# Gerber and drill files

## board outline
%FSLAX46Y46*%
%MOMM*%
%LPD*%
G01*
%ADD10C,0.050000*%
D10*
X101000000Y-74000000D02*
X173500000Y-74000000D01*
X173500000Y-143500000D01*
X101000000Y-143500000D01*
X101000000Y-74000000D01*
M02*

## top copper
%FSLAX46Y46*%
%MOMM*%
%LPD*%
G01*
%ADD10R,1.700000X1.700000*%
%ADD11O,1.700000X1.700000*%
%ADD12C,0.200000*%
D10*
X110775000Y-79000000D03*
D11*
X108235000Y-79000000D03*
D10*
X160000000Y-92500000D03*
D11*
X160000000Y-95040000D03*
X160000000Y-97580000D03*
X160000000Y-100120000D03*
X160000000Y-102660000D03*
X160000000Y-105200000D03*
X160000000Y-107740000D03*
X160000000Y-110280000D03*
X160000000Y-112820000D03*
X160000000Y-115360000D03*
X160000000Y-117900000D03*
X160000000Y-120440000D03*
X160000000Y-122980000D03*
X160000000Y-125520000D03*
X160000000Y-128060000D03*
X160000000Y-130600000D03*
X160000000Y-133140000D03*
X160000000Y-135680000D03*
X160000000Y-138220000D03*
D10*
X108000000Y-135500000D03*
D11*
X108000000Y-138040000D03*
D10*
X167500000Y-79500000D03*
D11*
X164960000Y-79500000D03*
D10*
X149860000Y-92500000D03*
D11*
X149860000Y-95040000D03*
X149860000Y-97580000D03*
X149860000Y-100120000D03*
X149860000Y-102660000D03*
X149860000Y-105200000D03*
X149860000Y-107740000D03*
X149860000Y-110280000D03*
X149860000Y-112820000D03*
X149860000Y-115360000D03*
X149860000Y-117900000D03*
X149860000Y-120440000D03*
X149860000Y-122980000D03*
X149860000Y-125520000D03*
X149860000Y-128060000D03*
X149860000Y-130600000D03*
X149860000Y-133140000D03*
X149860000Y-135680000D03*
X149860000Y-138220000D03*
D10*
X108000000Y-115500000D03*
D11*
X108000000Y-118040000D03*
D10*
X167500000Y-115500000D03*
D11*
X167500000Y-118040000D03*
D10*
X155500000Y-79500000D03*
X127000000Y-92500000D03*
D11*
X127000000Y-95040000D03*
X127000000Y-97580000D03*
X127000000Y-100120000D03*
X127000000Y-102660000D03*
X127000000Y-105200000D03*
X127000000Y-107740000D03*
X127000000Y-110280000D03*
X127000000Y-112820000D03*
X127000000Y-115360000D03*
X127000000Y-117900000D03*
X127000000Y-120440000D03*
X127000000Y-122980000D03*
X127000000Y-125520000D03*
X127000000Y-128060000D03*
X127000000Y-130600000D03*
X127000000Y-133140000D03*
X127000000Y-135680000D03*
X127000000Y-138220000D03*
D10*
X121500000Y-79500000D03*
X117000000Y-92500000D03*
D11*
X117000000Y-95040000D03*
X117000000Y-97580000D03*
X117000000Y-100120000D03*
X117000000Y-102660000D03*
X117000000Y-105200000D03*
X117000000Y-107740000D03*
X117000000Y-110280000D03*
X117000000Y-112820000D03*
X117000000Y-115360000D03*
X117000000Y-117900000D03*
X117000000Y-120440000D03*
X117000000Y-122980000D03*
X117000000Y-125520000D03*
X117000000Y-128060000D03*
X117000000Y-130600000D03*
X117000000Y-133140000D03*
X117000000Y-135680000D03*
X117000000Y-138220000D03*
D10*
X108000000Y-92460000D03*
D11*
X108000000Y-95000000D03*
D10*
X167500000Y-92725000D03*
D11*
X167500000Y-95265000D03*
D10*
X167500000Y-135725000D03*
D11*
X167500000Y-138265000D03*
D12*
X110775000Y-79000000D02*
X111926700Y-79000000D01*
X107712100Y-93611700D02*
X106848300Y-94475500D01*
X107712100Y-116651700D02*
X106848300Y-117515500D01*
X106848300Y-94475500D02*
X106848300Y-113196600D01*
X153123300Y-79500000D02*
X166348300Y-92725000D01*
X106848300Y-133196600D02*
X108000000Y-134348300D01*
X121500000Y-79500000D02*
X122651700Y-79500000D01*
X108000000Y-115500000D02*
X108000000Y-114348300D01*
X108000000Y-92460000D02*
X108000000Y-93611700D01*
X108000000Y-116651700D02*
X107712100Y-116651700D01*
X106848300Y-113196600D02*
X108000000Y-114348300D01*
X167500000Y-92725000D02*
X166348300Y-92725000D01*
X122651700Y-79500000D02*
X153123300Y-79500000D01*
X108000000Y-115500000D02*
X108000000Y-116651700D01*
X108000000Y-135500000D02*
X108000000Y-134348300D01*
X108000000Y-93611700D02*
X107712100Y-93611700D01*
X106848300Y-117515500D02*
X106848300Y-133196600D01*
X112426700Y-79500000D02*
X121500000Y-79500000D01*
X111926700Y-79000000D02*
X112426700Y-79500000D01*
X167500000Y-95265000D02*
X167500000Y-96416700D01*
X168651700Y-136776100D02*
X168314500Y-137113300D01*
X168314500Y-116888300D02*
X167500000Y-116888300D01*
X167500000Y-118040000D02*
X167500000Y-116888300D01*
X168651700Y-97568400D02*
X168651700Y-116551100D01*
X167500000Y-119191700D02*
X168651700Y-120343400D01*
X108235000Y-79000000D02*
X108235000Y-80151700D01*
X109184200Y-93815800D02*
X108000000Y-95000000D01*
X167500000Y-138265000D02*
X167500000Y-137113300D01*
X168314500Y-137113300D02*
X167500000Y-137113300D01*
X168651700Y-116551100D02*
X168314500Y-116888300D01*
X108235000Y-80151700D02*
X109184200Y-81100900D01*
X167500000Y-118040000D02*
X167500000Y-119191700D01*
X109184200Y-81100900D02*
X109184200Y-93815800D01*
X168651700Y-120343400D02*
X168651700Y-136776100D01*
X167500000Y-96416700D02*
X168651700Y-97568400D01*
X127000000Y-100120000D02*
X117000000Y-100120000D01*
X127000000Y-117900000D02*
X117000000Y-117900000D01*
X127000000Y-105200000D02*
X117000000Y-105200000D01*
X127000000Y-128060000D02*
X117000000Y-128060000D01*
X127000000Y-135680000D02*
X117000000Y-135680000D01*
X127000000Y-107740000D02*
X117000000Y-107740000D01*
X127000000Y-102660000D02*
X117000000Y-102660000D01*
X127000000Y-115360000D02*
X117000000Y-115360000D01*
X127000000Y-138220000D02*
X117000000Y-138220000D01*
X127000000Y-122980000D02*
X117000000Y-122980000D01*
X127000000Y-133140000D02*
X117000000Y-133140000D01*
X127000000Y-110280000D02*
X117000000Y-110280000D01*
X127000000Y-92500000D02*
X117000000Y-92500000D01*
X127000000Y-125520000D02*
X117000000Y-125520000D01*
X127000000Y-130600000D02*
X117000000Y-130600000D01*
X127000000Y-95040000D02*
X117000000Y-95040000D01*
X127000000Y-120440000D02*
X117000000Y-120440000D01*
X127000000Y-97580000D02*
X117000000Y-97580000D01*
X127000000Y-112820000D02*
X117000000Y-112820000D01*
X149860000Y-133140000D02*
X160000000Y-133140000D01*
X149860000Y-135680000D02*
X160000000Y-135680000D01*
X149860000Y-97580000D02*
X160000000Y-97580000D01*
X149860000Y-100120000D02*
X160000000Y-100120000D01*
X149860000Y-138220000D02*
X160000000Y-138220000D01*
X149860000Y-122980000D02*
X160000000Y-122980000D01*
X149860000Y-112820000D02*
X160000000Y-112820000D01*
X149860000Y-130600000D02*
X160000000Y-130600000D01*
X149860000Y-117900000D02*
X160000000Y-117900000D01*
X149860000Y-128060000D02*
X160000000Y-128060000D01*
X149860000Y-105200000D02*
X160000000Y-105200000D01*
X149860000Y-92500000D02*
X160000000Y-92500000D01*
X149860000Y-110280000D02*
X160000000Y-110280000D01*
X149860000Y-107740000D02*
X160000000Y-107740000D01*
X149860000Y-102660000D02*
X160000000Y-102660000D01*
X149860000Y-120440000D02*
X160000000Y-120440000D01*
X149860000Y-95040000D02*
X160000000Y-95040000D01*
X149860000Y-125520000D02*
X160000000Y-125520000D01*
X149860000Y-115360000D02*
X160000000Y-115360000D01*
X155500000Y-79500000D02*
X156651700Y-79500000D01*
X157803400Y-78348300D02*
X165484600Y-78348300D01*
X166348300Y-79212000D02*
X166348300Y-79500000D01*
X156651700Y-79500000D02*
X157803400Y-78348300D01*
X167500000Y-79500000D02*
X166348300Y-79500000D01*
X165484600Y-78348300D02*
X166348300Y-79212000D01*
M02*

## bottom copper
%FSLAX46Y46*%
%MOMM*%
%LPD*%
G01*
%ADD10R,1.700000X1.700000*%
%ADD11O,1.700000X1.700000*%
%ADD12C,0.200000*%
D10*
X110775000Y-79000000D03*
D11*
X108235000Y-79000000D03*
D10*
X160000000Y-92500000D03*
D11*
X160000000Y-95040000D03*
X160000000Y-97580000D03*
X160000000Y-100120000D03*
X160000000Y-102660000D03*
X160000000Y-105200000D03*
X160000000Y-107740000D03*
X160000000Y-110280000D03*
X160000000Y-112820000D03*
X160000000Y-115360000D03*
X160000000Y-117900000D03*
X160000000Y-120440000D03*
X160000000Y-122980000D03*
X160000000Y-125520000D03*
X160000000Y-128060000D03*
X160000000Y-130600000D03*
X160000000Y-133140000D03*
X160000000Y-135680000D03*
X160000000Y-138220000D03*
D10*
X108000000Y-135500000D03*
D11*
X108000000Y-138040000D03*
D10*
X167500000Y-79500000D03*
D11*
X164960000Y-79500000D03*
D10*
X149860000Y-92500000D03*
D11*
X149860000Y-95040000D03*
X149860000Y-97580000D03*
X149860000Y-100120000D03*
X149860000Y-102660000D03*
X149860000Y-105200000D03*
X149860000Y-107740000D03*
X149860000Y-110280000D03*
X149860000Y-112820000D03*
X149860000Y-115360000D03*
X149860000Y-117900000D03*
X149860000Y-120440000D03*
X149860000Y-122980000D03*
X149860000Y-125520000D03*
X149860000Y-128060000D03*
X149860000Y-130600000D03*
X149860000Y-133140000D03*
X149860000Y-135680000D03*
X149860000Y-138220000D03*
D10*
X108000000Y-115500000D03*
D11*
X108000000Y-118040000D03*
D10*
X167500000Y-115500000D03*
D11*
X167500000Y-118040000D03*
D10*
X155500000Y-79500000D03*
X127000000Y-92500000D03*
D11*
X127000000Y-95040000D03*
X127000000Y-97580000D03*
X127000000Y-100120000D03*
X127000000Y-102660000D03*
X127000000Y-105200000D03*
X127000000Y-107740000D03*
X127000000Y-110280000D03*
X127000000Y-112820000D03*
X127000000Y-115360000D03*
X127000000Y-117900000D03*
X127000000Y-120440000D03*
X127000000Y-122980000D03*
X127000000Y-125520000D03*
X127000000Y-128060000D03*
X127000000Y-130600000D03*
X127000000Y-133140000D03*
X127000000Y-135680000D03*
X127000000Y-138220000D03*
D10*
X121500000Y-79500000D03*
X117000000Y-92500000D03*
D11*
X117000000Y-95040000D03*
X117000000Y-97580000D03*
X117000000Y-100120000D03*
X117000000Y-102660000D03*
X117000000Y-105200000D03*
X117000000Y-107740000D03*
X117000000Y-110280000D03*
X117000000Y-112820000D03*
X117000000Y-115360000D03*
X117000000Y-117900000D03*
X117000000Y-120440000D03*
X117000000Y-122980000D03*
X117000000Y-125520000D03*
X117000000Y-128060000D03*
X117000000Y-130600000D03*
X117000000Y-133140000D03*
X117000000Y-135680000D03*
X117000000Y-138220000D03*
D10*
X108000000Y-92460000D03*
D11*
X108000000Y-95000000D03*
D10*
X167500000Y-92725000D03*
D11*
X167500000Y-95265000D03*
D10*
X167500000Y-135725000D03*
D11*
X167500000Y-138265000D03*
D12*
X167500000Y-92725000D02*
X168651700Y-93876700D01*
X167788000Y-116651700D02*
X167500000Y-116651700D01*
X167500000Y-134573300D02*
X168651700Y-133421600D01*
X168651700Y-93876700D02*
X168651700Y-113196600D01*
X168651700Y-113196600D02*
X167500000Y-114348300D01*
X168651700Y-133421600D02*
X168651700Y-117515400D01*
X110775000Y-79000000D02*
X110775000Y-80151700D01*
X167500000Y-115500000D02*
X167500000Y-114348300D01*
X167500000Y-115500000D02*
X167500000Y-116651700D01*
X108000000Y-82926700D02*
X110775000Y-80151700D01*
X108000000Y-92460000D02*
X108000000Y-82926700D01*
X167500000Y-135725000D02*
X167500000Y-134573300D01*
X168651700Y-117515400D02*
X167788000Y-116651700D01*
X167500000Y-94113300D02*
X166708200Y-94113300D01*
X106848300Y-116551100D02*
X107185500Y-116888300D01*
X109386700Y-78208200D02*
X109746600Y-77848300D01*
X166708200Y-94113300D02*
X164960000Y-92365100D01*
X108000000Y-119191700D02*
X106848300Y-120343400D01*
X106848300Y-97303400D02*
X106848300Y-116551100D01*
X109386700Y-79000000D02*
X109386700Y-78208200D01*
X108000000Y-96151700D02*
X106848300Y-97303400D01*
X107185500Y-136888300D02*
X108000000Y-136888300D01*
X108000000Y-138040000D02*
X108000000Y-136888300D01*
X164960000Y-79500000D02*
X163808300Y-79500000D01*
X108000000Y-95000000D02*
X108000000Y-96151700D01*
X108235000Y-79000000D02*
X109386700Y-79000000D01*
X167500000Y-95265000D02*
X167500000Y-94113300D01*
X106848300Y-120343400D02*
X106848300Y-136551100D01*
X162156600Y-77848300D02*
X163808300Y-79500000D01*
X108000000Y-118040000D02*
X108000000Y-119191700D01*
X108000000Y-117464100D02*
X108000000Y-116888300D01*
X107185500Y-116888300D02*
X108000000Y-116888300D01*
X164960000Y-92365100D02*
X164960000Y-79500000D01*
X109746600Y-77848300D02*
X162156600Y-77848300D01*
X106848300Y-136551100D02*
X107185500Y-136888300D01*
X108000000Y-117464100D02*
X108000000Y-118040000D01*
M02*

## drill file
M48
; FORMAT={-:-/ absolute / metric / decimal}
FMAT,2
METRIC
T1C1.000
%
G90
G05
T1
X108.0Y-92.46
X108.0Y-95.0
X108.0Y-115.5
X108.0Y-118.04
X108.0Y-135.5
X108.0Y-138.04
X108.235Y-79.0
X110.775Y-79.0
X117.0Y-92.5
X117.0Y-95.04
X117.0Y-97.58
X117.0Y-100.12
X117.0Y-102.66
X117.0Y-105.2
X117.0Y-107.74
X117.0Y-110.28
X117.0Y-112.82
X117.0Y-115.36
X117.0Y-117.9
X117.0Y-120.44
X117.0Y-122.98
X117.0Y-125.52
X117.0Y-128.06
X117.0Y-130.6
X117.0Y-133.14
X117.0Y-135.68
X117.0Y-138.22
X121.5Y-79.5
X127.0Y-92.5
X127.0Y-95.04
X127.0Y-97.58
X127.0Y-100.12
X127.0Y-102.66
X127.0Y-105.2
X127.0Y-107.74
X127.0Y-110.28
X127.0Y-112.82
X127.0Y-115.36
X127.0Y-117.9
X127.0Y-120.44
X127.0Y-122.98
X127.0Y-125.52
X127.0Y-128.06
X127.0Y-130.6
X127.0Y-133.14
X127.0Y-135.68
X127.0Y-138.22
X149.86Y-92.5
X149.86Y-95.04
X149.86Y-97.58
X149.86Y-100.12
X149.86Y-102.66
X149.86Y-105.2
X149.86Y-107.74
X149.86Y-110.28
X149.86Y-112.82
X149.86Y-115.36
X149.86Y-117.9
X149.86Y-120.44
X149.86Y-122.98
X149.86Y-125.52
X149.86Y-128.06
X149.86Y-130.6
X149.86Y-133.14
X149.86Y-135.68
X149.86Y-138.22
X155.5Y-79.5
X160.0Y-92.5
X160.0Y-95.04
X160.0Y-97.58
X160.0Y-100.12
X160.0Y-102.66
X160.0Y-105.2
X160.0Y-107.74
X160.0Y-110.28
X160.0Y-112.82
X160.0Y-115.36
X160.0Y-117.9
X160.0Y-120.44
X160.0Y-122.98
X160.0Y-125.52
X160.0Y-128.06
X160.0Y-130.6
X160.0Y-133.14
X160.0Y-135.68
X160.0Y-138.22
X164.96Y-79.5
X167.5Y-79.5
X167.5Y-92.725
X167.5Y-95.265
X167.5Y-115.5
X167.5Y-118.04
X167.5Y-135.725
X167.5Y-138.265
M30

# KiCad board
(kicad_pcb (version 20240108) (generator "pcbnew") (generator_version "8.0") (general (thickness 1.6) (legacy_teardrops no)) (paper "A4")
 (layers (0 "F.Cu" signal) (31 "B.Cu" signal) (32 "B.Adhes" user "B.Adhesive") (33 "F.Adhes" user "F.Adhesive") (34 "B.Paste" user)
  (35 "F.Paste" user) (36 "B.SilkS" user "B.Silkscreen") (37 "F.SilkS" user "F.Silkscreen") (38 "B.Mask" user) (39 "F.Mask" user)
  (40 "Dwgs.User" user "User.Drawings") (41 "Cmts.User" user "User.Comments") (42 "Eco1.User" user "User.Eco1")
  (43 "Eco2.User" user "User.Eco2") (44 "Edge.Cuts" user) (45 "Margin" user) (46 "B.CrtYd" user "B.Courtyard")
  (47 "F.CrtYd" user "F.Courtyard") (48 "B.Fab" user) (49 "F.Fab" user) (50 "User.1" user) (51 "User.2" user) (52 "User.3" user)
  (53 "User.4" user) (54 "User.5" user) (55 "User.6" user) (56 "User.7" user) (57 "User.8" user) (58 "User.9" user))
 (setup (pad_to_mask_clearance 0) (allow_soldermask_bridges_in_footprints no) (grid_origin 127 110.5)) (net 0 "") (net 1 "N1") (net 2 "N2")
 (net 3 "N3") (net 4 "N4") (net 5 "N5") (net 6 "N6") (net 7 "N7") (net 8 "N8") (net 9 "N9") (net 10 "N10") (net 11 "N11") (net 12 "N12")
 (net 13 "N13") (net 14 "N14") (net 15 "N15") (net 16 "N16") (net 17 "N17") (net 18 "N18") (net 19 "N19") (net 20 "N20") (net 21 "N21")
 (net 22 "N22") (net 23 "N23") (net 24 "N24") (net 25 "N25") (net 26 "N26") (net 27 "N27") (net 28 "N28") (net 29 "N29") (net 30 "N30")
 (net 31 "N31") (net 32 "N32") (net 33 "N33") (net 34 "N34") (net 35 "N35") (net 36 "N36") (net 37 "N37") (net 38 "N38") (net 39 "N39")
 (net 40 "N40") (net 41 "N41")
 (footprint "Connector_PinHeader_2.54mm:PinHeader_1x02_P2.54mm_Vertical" (layer "F.Cu") (at 110.775 79 -90)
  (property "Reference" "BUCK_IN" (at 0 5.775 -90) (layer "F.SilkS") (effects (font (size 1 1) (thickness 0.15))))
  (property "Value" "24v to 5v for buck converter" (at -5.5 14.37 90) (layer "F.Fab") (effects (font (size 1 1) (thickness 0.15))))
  (pad "1" thru_hole rect (at 0 0 270) (size 1.7 1.7) (drill 1) (layers "*.Cu" "*.Mask") (remove_unused_layers no) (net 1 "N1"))
  (pad "2" thru_hole oval (at 0 2.54 270) (size 1.7 1.7) (drill 1) (layers "*.Cu" "*.Mask") (remove_unused_layers no) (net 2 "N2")))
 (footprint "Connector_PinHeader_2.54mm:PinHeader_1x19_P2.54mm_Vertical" (layer "F.Cu") (at 160 92.5)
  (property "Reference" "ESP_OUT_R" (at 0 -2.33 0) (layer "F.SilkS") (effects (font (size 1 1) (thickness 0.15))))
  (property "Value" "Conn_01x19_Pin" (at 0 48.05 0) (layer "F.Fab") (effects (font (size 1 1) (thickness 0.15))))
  (pad "1" thru_hole rect (at 0 0) (size 1.7 1.7) (drill 1) (layers "*.Cu" "*.Mask") (remove_unused_layers no) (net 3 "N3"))
  (pad "2" thru_hole oval (at 0 2.54) (size 1.7 1.7) (drill 1) (layers "*.Cu" "*.Mask") (remove_unused_layers no) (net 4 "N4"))
  (pad "3" thru_hole oval (at 0 5.08) (size 1.7 1.7) (drill 1) (layers "*.Cu" "*.Mask") (remove_unused_layers no) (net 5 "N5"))
  (pad "4" thru_hole oval (at 0 7.62) (size 1.7 1.7) (drill 1) (layers "*.Cu" "*.Mask") (remove_unused_layers no) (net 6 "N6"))
  (pad "5" thru_hole oval (at 0 10.16) (size 1.7 1.7) (drill 1) (layers "*.Cu" "*.Mask") (remove_unused_layers no) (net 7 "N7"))
  (pad "6" thru_hole oval (at 0 12.7) (size 1.7 1.7) (drill 1) (layers "*.Cu" "*.Mask") (remove_unused_layers no) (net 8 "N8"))
  (pad "7" thru_hole oval (at 0 15.24) (size 1.7 1.7) (drill 1) (layers "*.Cu" "*.Mask") (remove_unused_layers no) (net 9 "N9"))
  (pad "8" thru_hole oval (at 0 17.78) (size 1.7 1.7) (drill 1) (layers "*.Cu" "*.Mask") (remove_unused_layers no) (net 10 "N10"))
  (pad "9" thru_hole oval (at 0 20.32) (size 1.7 1.7) (drill 1) (layers "*.Cu" "*.Mask") (remove_unused_layers no) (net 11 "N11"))
  (pad "10" thru_hole oval (at 0 22.86) (size 1.7 1.7) (drill 1) (layers "*.Cu" "*.Mask") (remove_unused_layers no) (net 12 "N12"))
  (pad "11" thru_hole oval (at 0 25.4) (size 1.7 1.7) (drill 1) (layers "*.Cu" "*.Mask") (remove_unused_layers no) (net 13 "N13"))
  (pad "12" thru_hole oval (at 0 27.94) (size 1.7 1.7) (drill 1) (layers "*.Cu" "*.Mask") (remove_unused_layers no) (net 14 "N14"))
  (pad "13" thru_hole oval (at 0 30.48) (size 1.7 1.7) (drill 1) (layers "*.Cu" "*.Mask") (remove_unused_layers no) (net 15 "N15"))
  (pad "14" thru_hole oval (at 0 33.02) (size 1.7 1.7) (drill 1) (layers "*.Cu" "*.Mask") (remove_unused_layers no) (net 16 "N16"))
  (pad "15" thru_hole oval (at 0 35.56) (size 1.7 1.7) (drill 1) (layers "*.Cu" "*.Mask") (remove_unused_layers no) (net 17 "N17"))
  (pad "16" thru_hole oval (at 0 38.1) (size 1.7 1.7) (drill 1) (layers "*.Cu" "*.Mask") (remove_unused_layers no) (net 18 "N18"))
  (pad "17" thru_hole oval (at 0 40.64) (size 1.7 1.7) (drill 1) (layers "*.Cu" "*.Mask") (remove_unused_layers no) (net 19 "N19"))
  (pad "18" thru_hole oval (at 0 43.18) (size 1.7 1.7) (drill 1) (layers "*.Cu" "*.Mask") (remove_unused_layers no) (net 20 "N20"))
  (pad "19" thru_hole oval (at 0 45.72) (size 1.7 1.7) (drill 1) (layers "*.Cu" "*.Mask") (remove_unused_layers no) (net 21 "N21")))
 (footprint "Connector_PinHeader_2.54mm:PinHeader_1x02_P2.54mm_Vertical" (layer "F.Cu") (at 108 135.5)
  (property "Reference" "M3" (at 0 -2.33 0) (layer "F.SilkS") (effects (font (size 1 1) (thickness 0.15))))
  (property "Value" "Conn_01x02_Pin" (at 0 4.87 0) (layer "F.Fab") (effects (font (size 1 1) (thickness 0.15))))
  (pad "1" thru_hole rect (at 0 0) (size 1.7 1.7) (drill 1) (layers "*.Cu" "*.Mask") (remove_unused_layers no) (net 1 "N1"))
  (pad "2" thru_hole oval (at 0 2.54) (size 1.7 1.7) (drill 1) (layers "*.Cu" "*.Mask") (remove_unused_layers no) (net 2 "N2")))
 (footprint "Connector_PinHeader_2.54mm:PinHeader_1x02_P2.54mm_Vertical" (layer "F.Cu") (at 167.5 79.5 -90)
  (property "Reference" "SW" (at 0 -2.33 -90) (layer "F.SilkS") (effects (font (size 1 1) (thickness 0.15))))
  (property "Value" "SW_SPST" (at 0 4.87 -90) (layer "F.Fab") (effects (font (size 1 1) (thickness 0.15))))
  (pad "1" thru_hole rect (at 0 0 270) (size 1.7 1.7) (drill 1) (layers "*.Cu" "*.Mask") (remove_unused_layers no) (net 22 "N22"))
  (pad "2" thru_hole oval (at 0 2.54 270) (size 1.7 1.7) (drill 1) (layers "*.Cu" "*.Mask") (remove_unused_layers no) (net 2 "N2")))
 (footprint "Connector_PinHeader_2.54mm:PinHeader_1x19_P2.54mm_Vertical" (layer "F.Cu") (at 149.86 92.5)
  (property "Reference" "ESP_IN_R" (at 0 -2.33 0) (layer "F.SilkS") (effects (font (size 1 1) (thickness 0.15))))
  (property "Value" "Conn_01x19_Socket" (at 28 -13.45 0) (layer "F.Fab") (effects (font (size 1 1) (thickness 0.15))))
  (pad "1" thru_hole rect (at 0 0) (size 1.7 1.7) (drill 1) (layers "*.Cu" "*.Mask") (remove_unused_layers no) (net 3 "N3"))
  (pad "2" thru_hole oval (at 0 2.54) (size 1.7 1.7) (drill 1) (layers "*.Cu" "*.Mask") (remove_unused_layers no) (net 4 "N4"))
  (pad "3" thru_hole oval (at 0 5.08) (size 1.7 1.7) (drill 1) (layers "*.Cu" "*.Mask") (remove_unused_layers no) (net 5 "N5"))
  (pad "4" thru_hole oval (at 0 7.62) (size 1.7 1.7) (drill 1) (layers "*.Cu" "*.Mask") (remove_unused_layers no) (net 6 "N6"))
  (pad "5" thru_hole oval (at 0 10.16) (size 1.7 1.7) (drill 1) (layers "*.Cu" "*.Mask") (remove_unused_layers no) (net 7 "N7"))
  (pad "6" thru_hole oval (at 0 12.7) (size 1.7 1.7) (drill 1) (layers "*.Cu" "*.Mask") (remove_unused_layers no) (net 8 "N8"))
  (pad "7" thru_hole oval (at 0 15.24) (size 1.7 1.7) (drill 1) (layers "*.Cu" "*.Mask") (remove_unused_layers no) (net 9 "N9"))
  (pad "8" thru_hole oval (at 0 17.78) (size 1.7 1.7) (drill 1) (layers "*.Cu" "*.Mask") (remove_unused_layers no) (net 10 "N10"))
  (pad "9" thru_hole oval (at 0 20.32) (size 1.7 1.7) (drill 1) (layers "*.Cu" "*.Mask") (remove_unused_layers no) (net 11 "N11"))
  (pad "10" thru_hole oval (at 0 22.86) (size 1.7 1.7) (drill 1) (layers "*.Cu" "*.Mask") (remove_unused_layers no) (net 12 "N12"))
  (pad "11" thru_hole oval (at 0 25.4) (size 1.7 1.7) (drill 1) (layers "*.Cu" "*.Mask") (remove_unused_layers no) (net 13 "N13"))
  (pad "12" thru_hole oval (at 0 27.94) (size 1.7 1.7) (drill 1) (layers "*.Cu" "*.Mask") (remove_unused_layers no) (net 14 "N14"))
  (pad "13" thru_hole oval (at 0 30.48) (size 1.7 1.7) (drill 1) (layers "*.Cu" "*.Mask") (remove_unused_layers no) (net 15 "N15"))
  (pad "14" thru_hole oval (at 0 33.02) (size 1.7 1.7) (drill 1) (layers "*.Cu" "*.Mask") (remove_unused_layers no) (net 16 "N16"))
  (pad "15" thru_hole oval (at 0 35.56) (size 1.7 1.7) (drill 1) (layers "*.Cu" "*.Mask") (remove_unused_layers no) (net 17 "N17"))
  (pad "16" thru_hole oval (at 0 38.1) (size 1.7 1.7) (drill 1) (layers "*.Cu" "*.Mask") (remove_unused_layers no) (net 18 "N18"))
  (pad "17" thru_hole oval (at 0 40.64) (size 1.7 1.7) (drill 1) (layers "*.Cu" "*.Mask") (remove_unused_layers no) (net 19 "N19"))
  (pad "18" thru_hole oval (at 0 43.18) (size 1.7 1.7) (drill 1) (layers "*.Cu" "*.Mask") (remove_unused_layers no) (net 20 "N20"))
  (pad "19" thru_hole oval (at 0 45.72) (size 1.7 1.7) (drill 1) (layers "*.Cu" "*.Mask") (remove_unused_layers no) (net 21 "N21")))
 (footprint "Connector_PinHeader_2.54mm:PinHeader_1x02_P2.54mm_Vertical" (layer "F.Cu") (at 108 115.5)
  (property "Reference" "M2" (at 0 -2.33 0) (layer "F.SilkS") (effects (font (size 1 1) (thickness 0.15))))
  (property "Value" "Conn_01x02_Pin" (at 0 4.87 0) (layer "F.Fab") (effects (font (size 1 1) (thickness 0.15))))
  (pad "1" thru_hole rect (at 0 0) (size 1.7 1.7) (drill 1) (layers "*.Cu" "*.Mask") (remove_unused_layers no) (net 1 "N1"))
  (pad "2" thru_hole oval (at 0 2.54) (size 1.7 1.7) (drill 1) (layers "*.Cu" "*.Mask") (remove_unused_layers no) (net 2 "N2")))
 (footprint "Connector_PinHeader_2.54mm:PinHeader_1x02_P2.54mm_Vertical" (layer "F.Cu") (at 167.5 115.5)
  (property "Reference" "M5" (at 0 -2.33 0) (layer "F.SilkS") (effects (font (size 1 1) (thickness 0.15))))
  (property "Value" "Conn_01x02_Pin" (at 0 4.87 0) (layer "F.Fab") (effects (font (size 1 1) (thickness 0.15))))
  (pad "1" thru_hole rect (at 0 0) (size 1.7 1.7) (drill 1) (layers "*.Cu" "*.Mask") (remove_unused_layers no) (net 1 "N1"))
  (pad "2" thru_hole oval (at 0 2.54) (size 1.7 1.7) (drill 1) (layers "*.Cu" "*.Mask") (remove_unused_layers no) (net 2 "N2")))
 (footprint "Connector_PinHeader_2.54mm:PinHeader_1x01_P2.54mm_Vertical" (layer "F.Cu") (at 155.5 79.5 180)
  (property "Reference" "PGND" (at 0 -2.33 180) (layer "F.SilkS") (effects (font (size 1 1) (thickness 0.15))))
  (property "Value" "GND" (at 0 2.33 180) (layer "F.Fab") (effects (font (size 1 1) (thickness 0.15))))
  (pad "1" thru_hole rect (at 0 0 180) (size 1.7 1.7) (drill 1) (layers "*.Cu" "*.Mask") (remove_unused_layers no) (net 22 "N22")))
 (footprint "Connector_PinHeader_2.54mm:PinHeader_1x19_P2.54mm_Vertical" (layer "F.Cu") (at 127 92.5)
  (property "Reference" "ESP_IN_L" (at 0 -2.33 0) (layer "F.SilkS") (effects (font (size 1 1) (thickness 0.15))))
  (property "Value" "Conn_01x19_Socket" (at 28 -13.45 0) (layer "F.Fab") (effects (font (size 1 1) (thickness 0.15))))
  (pad "1" thru_hole rect (at 0 0) (size 1.7 1.7) (drill 1) (layers "*.Cu" "*.Mask") (remove_unused_layers no) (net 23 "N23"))
  (pad "2" thru_hole oval (at 0 2.54) (size 1.7 1.7) (drill 1) (layers "*.Cu" "*.Mask") (remove_unused_layers no) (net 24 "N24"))
  (pad "3" thru_hole oval (at 0 5.08) (size 1.7 1.7) (drill 1) (layers "*.Cu" "*.Mask") (remove_unused_layers no) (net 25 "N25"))
  (pad "4" thru_hole oval (at 0 7.62) (size 1.7 1.7) (drill 1) (layers "*.Cu" "*.Mask") (remove_unused_layers no) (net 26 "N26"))
  (pad "5" thru_hole oval (at 0 10.16) (size 1.7 1.7) (drill 1) (layers "*.Cu" "*.Mask") (remove_unused_layers no) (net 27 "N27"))
  (pad "6" thru_hole oval (at 0 12.7) (size 1.7 1.7) (drill 1) (layers "*.Cu" "*.Mask") (remove_unused_layers no) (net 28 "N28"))
  (pad "7" thru_hole oval (at 0 15.24) (size 1.7 1.7) (drill 1) (layers "*.Cu" "*.Mask") (remove_unused_layers no) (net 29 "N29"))
  (pad "8" thru_hole oval (at 0 17.78) (size 1.7 1.7) (drill 1) (layers "*.Cu" "*.Mask") (remove_unused_layers no) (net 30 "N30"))
  (pad "9" thru_hole oval (at 0 20.32) (size 1.7 1.7) (drill 1) (layers "*.Cu" "*.Mask") (remove_unused_layers no) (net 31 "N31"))
  (pad "10" thru_hole oval (at 0 22.86) (size 1.7 1.7) (drill 1) (layers "*.Cu" "*.Mask") (remove_unused_layers no) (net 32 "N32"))
  (pad "11" thru_hole oval (at 0 25.4) (size 1.7 1.7) (drill 1) (layers "*.Cu" "*.Mask") (remove_unused_layers no) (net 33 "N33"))
  (pad "12" thru_hole oval (at 0 27.94) (size 1.7 1.7) (drill 1) (layers "*.Cu" "*.Mask") (remove_unused_layers no) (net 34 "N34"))
  (pad "13" thru_hole oval (at 0 30.48) (size 1.7 1.7) (drill 1) (layers "*.Cu" "*.Mask") (remove_unused_layers no) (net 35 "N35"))
  (pad "14" thru_hole oval (at 0 33.02) (size 1.7 1.7) (drill 1) (layers "*.Cu" "*.Mask") (remove_unused_layers no) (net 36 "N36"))
  (pad "15" thru_hole oval (at 0 35.56) (size 1.7 1.7) (drill 1) (layers "*.Cu" "*.Mask") (remove_unused_layers no) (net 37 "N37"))
  (pad "16" thru_hole oval (at 0 38.1) (size 1.7 1.7) (drill 1) (layers "*.Cu" "*.Mask") (remove_unused_layers no) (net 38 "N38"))
  (pad "17" thru_hole oval (at 0 40.64) (size 1.7 1.7) (drill 1) (layers "*.Cu" "*.Mask") (remove_unused_layers no) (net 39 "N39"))
  (pad "18" thru_hole oval (at 0 43.18) (size 1.7 1.7) (drill 1) (layers "*.Cu" "*.Mask") (remove_unused_layers no) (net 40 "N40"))
  (pad "19" thru_hole oval (at 0 45.72) (size 1.7 1.7) (drill 1) (layers "*.Cu" "*.Mask") (remove_unused_layers no) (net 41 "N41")))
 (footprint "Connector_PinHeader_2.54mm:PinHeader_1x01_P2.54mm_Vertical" (layer "F.Cu") (at 121.5 79.5 180)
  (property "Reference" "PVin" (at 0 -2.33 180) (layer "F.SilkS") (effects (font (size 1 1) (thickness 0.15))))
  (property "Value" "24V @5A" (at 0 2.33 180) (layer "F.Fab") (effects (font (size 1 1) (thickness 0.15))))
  (pad "1" thru_hole rect (at 0 0 180) (size 1.7 1.7) (drill 1) (layers "*.Cu" "*.Mask") (remove_unused_layers no) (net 1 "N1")))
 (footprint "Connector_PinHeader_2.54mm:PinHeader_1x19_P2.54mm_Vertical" (layer "F.Cu") (at 117 92.5)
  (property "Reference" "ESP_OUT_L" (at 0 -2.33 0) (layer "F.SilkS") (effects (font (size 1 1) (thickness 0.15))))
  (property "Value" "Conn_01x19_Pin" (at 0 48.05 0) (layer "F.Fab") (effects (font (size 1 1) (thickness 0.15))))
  (pad "1" thru_hole rect (at 0 0) (size 1.7 1.7) (drill 1) (layers "*.Cu" "*.Mask") (remove_unused_layers no) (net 23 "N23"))
  (pad "2" thru_hole oval (at 0 2.54) (size 1.7 1.7) (drill 1) (layers "*.Cu" "*.Mask") (remove_unused_layers no) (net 24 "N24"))
  (pad "3" thru_hole oval (at 0 5.08) (size 1.7 1.7) (drill 1) (layers "*.Cu" "*.Mask") (remove_unused_layers no) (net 25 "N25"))
  (pad "4" thru_hole oval (at 0 7.62) (size 1.7 1.7) (drill 1) (layers "*.Cu" "*.Mask") (remove_unused_layers no) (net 26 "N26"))
  (pad "5" thru_hole oval (at 0 10.16) (size 1.7 1.7) (drill 1) (layers "*.Cu" "*.Mask") (remove_unused_layers no) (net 27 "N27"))
  (pad "6" thru_hole oval (at 0 12.7) (size 1.7 1.7) (drill 1) (layers "*.Cu" "*.Mask") (remove_unused_layers no) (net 28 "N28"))
  (pad "7" thru_hole oval (at 0 15.24) (size 1.7 1.7) (drill 1) (layers "*.Cu" "*.Mask") (remove_unused_layers no) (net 29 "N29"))
  (pad "8" thru_hole oval (at 0 17.78) (size 1.7 1.7) (drill 1) (layers "*.Cu" "*.Mask") (remove_unused_layers no) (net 30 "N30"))
  (pad "9" thru_hole oval (at 0 20.32) (size 1.7 1.7) (drill 1) (layers "*.Cu" "*.Mask") (remove_unused_layers no) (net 31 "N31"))
  (pad "10" thru_hole oval (at 0 22.86) (size 1.7 1.7) (drill 1) (layers "*.Cu" "*.Mask") (remove_unused_layers no) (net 32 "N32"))
  (pad "11" thru_hole oval (at 0 25.4) (size 1.7 1.7) (drill 1) (layers "*.Cu" "*.Mask") (remove_unused_layers no) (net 33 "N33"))
  (pad "12" thru_hole oval (at 0 27.94) (size 1.7 1.7) (drill 1) (layers "*.Cu" "*.Mask") (remove_unused_layers no) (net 34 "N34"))
  (pad "13" thru_hole oval (at 0 30.48) (size 1.7 1.7) (drill 1) (layers "*.Cu" "*.Mask") (remove_unused_layers no) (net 35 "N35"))
  (pad "14" thru_hole oval (at 0 33.02) (size 1.7 1.7) (drill 1) (layers "*.Cu" "*.Mask") (remove_unused_layers no) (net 36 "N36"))
  (pad "15" thru_hole oval (at 0 35.56) (size 1.7 1.7) (drill 1) (layers "*.Cu" "*.Mask") (remove_unused_layers no) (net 37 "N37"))
  (pad "16" thru_hole oval (at 0 38.1) (size 1.7 1.7) (drill 1) (layers "*.Cu" "*.Mask") (remove_unused_layers no) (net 38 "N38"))
  (pad "17" thru_hole oval (at 0 40.64) (size 1.7 1.7) (drill 1) (layers "*.Cu" "*.Mask") (remove_unused_layers no) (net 39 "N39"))
  (pad "18" thru_hole oval (at 0 43.18) (size 1.7 1.7) (drill 1) (layers "*.Cu" "*.Mask") (remove_unused_layers no) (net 40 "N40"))
  (pad "19" thru_hole oval (at 0 45.72) (size 1.7 1.7) (drill 1) (layers "*.Cu" "*.Mask") (remove_unused_layers no) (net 41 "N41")))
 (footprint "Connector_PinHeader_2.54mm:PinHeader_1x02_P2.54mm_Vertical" (layer "F.Cu") (at 108 92.46)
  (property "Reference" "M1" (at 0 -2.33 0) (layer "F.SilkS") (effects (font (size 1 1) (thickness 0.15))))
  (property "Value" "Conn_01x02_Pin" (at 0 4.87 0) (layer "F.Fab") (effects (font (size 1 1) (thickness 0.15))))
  (pad "1" thru_hole rect (at 0 0) (size 1.7 1.7) (drill 1) (layers "*.Cu" "*.Mask") (remove_unused_layers no) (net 1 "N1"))
  (pad "2" thru_hole oval (at 0 2.54) (size 1.7 1.7) (drill 1) (layers "*.Cu" "*.Mask") (remove_unused_layers no) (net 2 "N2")))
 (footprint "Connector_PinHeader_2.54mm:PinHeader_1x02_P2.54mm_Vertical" (layer "F.Cu") (at 167.5 92.725)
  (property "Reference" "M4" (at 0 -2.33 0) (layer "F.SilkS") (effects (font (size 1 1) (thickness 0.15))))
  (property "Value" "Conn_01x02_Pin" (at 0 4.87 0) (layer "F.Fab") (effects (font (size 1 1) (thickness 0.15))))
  (pad "1" thru_hole rect (at 0 0) (size 1.7 1.7) (drill 1) (layers "*.Cu" "*.Mask") (remove_unused_layers no) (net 1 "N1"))
  (pad "2" thru_hole oval (at 0 2.54) (size 1.7 1.7) (drill 1) (layers "*.Cu" "*.Mask") (remove_unused_layers no) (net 2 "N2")))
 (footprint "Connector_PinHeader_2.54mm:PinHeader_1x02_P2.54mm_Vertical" (layer "F.Cu") (at 167.5 135.725)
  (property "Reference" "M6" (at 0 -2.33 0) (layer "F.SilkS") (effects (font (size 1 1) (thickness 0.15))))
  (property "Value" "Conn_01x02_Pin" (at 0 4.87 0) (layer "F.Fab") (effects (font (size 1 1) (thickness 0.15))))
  (pad "1" thru_hole rect (at 0 0) (size 1.7 1.7) (drill 1) (layers "*.Cu" "*.Mask") (remove_unused_layers no) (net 1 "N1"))
  (pad "2" thru_hole oval (at 0 2.54) (size 1.7 1.7) (drill 1) (layers "*.Cu" "*.Mask") (remove_unused_layers no) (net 2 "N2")))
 (gr_rect (start 101 74) (end 173.5 143.5) (stroke (width 0.05) (type default)) (fill none) (layer "Edge.Cuts"))
 (segment (start 110.775 79) (end 111.9267 79) (width 0.2) (layer "F.Cu") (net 1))
 (segment (start 107.7121 93.6117) (end 106.8483 94.4755) (width 0.2) (layer "F.Cu") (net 1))
 (segment (start 107.7121 116.6517) (end 106.8483 117.5155) (width 0.2) (layer "F.Cu") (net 1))
 (segment (start 106.8483 94.4755) (end 106.8483 113.1966) (width 0.2) (layer "F.Cu") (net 1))
 (segment (start 153.1233 79.5) (end 166.3483 92.725) (width 0.2) (layer "F.Cu") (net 1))
 (segment (start 106.8483 133.1966) (end 108 134.3483) (width 0.2) (layer "F.Cu") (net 1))
 (segment (start 121.5 79.5) (end 122.6517 79.5) (width 0.2) (layer "F.Cu") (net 1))
 (segment (start 108 115.5) (end 108 114.3483) (width 0.2) (layer "F.Cu") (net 1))
 (segment (start 108 92.46) (end 108 93.6117) (width 0.2) (layer "F.Cu") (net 1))
 (segment (start 108 116.6517) (end 107.7121 116.6517) (width 0.2) (layer "F.Cu") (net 1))
 (segment (start 106.8483 113.1966) (end 108 114.3483) (width 0.2) (layer "F.Cu") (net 1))
 (segment (start 167.5 92.725) (end 166.3483 92.725) (width 0.2) (layer "F.Cu") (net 1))
 (segment (start 122.6517 79.5) (end 153.1233 79.5) (width 0.2) (layer "F.Cu") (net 1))
 (segment (start 108 115.5) (end 108 116.6517) (width 0.2) (layer "F.Cu") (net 1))
 (segment (start 108 135.5) (end 108 134.3483) (width 0.2) (layer "F.Cu") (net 1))
 (segment (start 108 93.6117) (end 107.7121 93.6117) (width 0.2) (layer "F.Cu") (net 1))
 (segment (start 106.8483 117.5155) (end 106.8483 133.1966) (width 0.2) (layer "F.Cu") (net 1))
 (segment (start 112.4267 79.5) (end 121.5 79.5) (width 0.2) (layer "F.Cu") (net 1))
 (segment (start 111.9267 79) (end 112.4267 79.5) (width 0.2) (layer "F.Cu") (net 1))
 (segment (start 167.5 92.725) (end 168.6517 93.8767) (width 0.2) (layer "B.Cu") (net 1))
 (segment (start 167.788 116.6517) (end 167.5 116.6517) (width 0.2) (layer "B.Cu") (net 1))
 (segment (start 167.5 134.5733) (end 168.6517 133.4216) (width 0.2) (layer "B.Cu") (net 1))
 (segment (start 168.6517 93.8767) (end 168.6517 113.1966) (width 0.2) (layer "B.Cu") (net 1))
 (segment (start 168.6517 113.1966) (end 167.5 114.3483) (width 0.2) (layer "B.Cu") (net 1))
 (segment (start 168.6517 133.4216) (end 168.6517 117.5154) (width 0.2) (layer "B.Cu") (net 1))
 (segment (start 110.775 79) (end 110.775 80.1517) (width 0.2) (layer "B.Cu") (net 1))
 (segment (start 167.5 115.5) (end 167.5 114.3483) (width 0.2) (layer "B.Cu") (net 1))
 (segment (start 167.5 115.5) (end 167.5 116.6517) (width 0.2) (layer "B.Cu") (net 1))
 (segment (start 108 82.9267) (end 110.775 80.1517) (width 0.2) (layer "B.Cu") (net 1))
 (segment (start 108 92.46) (end 108 82.9267) (width 0.2) (layer "B.Cu") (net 1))
 (segment (start 167.5 135.725) (end 167.5 134.5733) (width 0.2) (layer "B.Cu") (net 1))
 (segment (start 168.6517 117.5154) (end 167.788 116.6517) (width 0.2) (layer "B.Cu") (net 1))
 (segment (start 167.5 95.265) (end 167.5 96.4167) (width 0.2) (layer "F.Cu") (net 2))
 (segment (start 168.6517 136.7761) (end 168.3145 137.1133) (width 0.2) (layer "F.Cu") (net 2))
 (segment (start 168.3145 116.8883) (end 167.5 116.8883) (width 0.2) (layer "F.Cu") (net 2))
 (segment (start 167.5 118.04) (end 167.5 116.8883) (width 0.2) (layer "F.Cu") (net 2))
 (segment (start 168.6517 97.5684) (end 168.6517 116.5511) (width 0.2) (layer "F.Cu") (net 2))
 (segment (start 167.5 119.1917) (end 168.6517 120.3434) (width 0.2) (layer "F.Cu") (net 2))
 (segment (start 108.235 79) (end 108.235 80.1517) (width 0.2) (layer "F.Cu") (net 2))
 (segment (start 109.1842 93.8158) (end 108 95) (width 0.2) (layer "F.Cu") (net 2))
 (segment (start 167.5 138.265) (end 167.5 137.1133) (width 0.2) (layer "F.Cu") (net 2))
 (segment (start 168.3145 137.1133) (end 167.5 137.1133) (width 0.2) (layer "F.Cu") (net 2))
 (segment (start 168.6517 116.5511) (end 168.3145 116.8883) (width 0.2) (layer "F.Cu") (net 2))
 (segment (start 108.235 80.1517) (end 109.1842 81.1009) (width 0.2) (layer "F.Cu") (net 2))
 (segment (start 167.5 118.04) (end 167.5 119.1917) (width 0.2) (layer "F.Cu") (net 2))
 (segment (start 109.1842 81.1009) (end 109.1842 93.8158) (width 0.2) (layer "F.Cu") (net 2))
 (segment (start 168.6517 120.3434) (end 168.6517 136.7761) (width 0.2) (layer "F.Cu") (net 2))
 (segment (start 167.5 96.4167) (end 168.6517 97.5684) (width 0.2) (layer "F.Cu") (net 2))
 (segment (start 167.5 94.1133) (end 166.7082 94.1133) (width 0.2) (layer "B.Cu") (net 2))
 (segment (start 106.8483 116.5511) (end 107.1855 116.8883) (width 0.2) (layer "B.Cu") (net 2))
 (segment (start 109.3867 78.2082) (end 109.7466 77.8483) (width 0.2) (layer "B.Cu") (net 2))
 (segment (start 166.7082 94.1133) (end 164.96 92.3651) (width 0.2) (layer "B.Cu") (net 2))
 (segment (start 108 119.1917) (end 106.8483 120.3434) (width 0.2) (layer "B.Cu") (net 2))
 (segment (start 106.8483 97.3034) (end 106.8483 116.5511) (width 0.2) (layer "B.Cu") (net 2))
 (segment (start 109.3867 79) (end 109.3867 78.2082) (width 0.2) (layer "B.Cu") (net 2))
 (segment (start 108 96.1517) (end 106.8483 97.3034) (width 0.2) (layer "B.Cu") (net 2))
 (segment (start 107.1855 136.8883) (end 108 136.8883) (width 0.2) (layer "B.Cu") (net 2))
 (segment (start 108 138.04) (end 108 136.8883) (width 0.2) (layer "B.Cu") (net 2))
 (segment (start 164.96 79.5) (end 163.8083 79.5) (width 0.2) (layer "B.Cu") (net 2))
 (segment (start 108 95) (end 108 96.1517) (width 0.2) (layer "B.Cu") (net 2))
 (segment (start 108.235 79) (end 109.3867 79) (width 0.2) (layer "B.Cu") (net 2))
 (segment (start 167.5 95.265) (end 167.5 94.1133) (width 0.2) (layer "B.Cu") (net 2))
 (segment (start 106.8483 120.3434) (end 106.8483 136.5511) (width 0.2) (layer "B.Cu") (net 2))
 (segment (start 162.1566 77.8483) (end 163.8083 79.5) (width 0.2) (layer "B.Cu") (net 2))
 (segment (start 108 118.04) (end 108 119.1917) (width 0.2) (layer "B.Cu") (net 2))
 (segment (start 108 117.4641) (end 108 116.8883) (width 0.2) (layer "B.Cu") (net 2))
 (segment (start 107.1855 116.8883) (end 108 116.8883) (width 0.2) (layer "B.Cu") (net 2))
 (segment (start 164.96 92.3651) (end 164.96 79.5) (width 0.2) (layer "B.Cu") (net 2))
 (segment (start 109.7466 77.8483) (end 162.1566 77.8483) (width 0.2) (layer "B.Cu") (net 2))
 (segment (start 106.8483 136.5511) (end 107.1855 136.8883) (width 0.2) (layer "B.Cu") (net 2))
 (segment (start 108 117.4641) (end 108 118.04) (width 0.2) (layer "B.Cu") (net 2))
 (segment (start 127 100.12) (end 117 100.12) (width 0.2) (layer "F.Cu") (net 26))
 (segment (start 127 117.9) (end 117 117.9) (width 0.2) (layer "F.Cu") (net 33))
 (segment (start 127 105.2) (end 117 105.2) (width 0.2) (layer "F.Cu") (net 28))
 (segment (start 127 128.06) (end 117 128.06) (width 0.2) (layer "F.Cu") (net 37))
 (segment (start 127 135.68) (end 117 135.68) (width 0.2) (layer "F.Cu") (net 40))
 (segment (start 127 107.74) (end 117 107.74) (width 0.2) (layer "F.Cu") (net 29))
 (segment (start 127 102.66) (end 117 102.66) (width 0.2) (layer "F.Cu") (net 27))
 (segment (start 127 115.36) (end 117 115.36) (width 0.2) (layer "F.Cu") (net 32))
 (segment (start 127 138.22) (end 117 138.22) (width 0.2) (layer "F.Cu") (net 41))
 (segment (start 127 122.98) (end 117 122.98) (width 0.2) (layer "F.Cu") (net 35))
 (segment (start 127 133.14) (end 117 133.14) (width 0.2) (layer "F.Cu") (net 39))
 (segment (start 127 110.28) (end 117 110.28) (width 0.2) (layer "F.Cu") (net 30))
 (segment (start 127 92.5) (end 117 92.5) (width 0.2) (layer "F.Cu") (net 23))
 (segment (start 127 125.52) (end 117 125.52) (width 0.2) (layer "F.Cu") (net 36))
 (segment (start 127 130.6) (end 117 130.6) (width 0.2) (layer "F.Cu") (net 38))
 (segment (start 127 95.04) (end 117 95.04) (width 0.2) (layer "F.Cu") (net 24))
 (segment (start 127 120.44) (end 117 120.44) (width 0.2) (layer "F.Cu") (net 34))
 (segment (start 127 97.58) (end 117 97.58) (width 0.2) (layer "F.Cu") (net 25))
 (segment (start 127 112.82) (end 117 112.82) (width 0.2) (layer "F.Cu") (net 31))
 (segment (start 149.86 133.14) (end 160 133.14) (width 0.2) (layer "F.Cu") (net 19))
 (segment (start 149.86 135.68) (end 160 135.68) (width 0.2) (layer "F.Cu") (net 20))
 (segment (start 149.86 97.58) (end 160 97.58) (width 0.2) (layer "F.Cu") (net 5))
 (segment (start 149.86 100.12) (end 160 100.12) (width 0.2) (layer "F.Cu") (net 6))
 (segment (start 149.86 138.22) (end 160 138.22) (width 0.2) (layer "F.Cu") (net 21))
 (segment (start 149.86 122.98) (end 160 122.98) (width 0.2) (layer "F.Cu") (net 15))
 (segment (start 149.86 112.82) (end 160 112.82) (width 0.2) (layer "F.Cu") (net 11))
 (segment (start 149.86 130.6) (end 160 130.6) (width 0.2) (layer "F.Cu") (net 18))
 (segment (start 149.86 117.9) (end 160 117.9) (width 0.2) (layer "F.Cu") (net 13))
 (segment (start 149.86 128.06) (end 160 128.06) (width 0.2) (layer "F.Cu") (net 17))
 (segment (start 149.86 105.2) (end 160 105.2) (width 0.2) (layer "F.Cu") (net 8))
 (segment (start 149.86 92.5) (end 160 92.5) (width 0.2) (layer "F.Cu") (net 3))
 (segment (start 149.86 110.28) (end 160 110.28) (width 0.2) (layer "F.Cu") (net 10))
 (segment (start 149.86 107.74) (end 160 107.74) (width 0.2) (layer "F.Cu") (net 9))
 (segment (start 149.86 102.66) (end 160 102.66) (width 0.2) (layer "F.Cu") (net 7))
 (segment (start 149.86 120.44) (end 160 120.44) (width 0.2) (layer "F.Cu") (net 14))
 (segment (start 149.86 95.04) (end 160 95.04) (width 0.2) (layer "F.Cu") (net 4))
 (segment (start 149.86 125.52) (end 160 125.52) (width 0.2) (layer "F.Cu") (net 16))
 (segment (start 149.86 115.36) (end 160 115.36) (width 0.2) (layer "F.Cu") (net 12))
 (segment (start 155.5 79.5) (end 156.6517 79.5) (width 0.2) (layer "F.Cu") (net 22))
 (segment (start 157.8034 78.3483) (end 165.4846 78.3483) (width 0.2) (layer "F.Cu") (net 22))
 (segment (start 166.3483 79.212) (end 166.3483 79.5) (width 0.2) (layer "F.Cu") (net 22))
 (segment (start 156.6517 79.5) (end 157.8034 78.3483) (width 0.2) (layer "F.Cu") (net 22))
 (segment (start 167.5 79.5) (end 166.3483 79.5) (width 0.2) (layer "F.Cu") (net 22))
 (segment (start 165.4846 78.3483) (end 166.3483 79.212) (width 0.2) (layer "F.Cu") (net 22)))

